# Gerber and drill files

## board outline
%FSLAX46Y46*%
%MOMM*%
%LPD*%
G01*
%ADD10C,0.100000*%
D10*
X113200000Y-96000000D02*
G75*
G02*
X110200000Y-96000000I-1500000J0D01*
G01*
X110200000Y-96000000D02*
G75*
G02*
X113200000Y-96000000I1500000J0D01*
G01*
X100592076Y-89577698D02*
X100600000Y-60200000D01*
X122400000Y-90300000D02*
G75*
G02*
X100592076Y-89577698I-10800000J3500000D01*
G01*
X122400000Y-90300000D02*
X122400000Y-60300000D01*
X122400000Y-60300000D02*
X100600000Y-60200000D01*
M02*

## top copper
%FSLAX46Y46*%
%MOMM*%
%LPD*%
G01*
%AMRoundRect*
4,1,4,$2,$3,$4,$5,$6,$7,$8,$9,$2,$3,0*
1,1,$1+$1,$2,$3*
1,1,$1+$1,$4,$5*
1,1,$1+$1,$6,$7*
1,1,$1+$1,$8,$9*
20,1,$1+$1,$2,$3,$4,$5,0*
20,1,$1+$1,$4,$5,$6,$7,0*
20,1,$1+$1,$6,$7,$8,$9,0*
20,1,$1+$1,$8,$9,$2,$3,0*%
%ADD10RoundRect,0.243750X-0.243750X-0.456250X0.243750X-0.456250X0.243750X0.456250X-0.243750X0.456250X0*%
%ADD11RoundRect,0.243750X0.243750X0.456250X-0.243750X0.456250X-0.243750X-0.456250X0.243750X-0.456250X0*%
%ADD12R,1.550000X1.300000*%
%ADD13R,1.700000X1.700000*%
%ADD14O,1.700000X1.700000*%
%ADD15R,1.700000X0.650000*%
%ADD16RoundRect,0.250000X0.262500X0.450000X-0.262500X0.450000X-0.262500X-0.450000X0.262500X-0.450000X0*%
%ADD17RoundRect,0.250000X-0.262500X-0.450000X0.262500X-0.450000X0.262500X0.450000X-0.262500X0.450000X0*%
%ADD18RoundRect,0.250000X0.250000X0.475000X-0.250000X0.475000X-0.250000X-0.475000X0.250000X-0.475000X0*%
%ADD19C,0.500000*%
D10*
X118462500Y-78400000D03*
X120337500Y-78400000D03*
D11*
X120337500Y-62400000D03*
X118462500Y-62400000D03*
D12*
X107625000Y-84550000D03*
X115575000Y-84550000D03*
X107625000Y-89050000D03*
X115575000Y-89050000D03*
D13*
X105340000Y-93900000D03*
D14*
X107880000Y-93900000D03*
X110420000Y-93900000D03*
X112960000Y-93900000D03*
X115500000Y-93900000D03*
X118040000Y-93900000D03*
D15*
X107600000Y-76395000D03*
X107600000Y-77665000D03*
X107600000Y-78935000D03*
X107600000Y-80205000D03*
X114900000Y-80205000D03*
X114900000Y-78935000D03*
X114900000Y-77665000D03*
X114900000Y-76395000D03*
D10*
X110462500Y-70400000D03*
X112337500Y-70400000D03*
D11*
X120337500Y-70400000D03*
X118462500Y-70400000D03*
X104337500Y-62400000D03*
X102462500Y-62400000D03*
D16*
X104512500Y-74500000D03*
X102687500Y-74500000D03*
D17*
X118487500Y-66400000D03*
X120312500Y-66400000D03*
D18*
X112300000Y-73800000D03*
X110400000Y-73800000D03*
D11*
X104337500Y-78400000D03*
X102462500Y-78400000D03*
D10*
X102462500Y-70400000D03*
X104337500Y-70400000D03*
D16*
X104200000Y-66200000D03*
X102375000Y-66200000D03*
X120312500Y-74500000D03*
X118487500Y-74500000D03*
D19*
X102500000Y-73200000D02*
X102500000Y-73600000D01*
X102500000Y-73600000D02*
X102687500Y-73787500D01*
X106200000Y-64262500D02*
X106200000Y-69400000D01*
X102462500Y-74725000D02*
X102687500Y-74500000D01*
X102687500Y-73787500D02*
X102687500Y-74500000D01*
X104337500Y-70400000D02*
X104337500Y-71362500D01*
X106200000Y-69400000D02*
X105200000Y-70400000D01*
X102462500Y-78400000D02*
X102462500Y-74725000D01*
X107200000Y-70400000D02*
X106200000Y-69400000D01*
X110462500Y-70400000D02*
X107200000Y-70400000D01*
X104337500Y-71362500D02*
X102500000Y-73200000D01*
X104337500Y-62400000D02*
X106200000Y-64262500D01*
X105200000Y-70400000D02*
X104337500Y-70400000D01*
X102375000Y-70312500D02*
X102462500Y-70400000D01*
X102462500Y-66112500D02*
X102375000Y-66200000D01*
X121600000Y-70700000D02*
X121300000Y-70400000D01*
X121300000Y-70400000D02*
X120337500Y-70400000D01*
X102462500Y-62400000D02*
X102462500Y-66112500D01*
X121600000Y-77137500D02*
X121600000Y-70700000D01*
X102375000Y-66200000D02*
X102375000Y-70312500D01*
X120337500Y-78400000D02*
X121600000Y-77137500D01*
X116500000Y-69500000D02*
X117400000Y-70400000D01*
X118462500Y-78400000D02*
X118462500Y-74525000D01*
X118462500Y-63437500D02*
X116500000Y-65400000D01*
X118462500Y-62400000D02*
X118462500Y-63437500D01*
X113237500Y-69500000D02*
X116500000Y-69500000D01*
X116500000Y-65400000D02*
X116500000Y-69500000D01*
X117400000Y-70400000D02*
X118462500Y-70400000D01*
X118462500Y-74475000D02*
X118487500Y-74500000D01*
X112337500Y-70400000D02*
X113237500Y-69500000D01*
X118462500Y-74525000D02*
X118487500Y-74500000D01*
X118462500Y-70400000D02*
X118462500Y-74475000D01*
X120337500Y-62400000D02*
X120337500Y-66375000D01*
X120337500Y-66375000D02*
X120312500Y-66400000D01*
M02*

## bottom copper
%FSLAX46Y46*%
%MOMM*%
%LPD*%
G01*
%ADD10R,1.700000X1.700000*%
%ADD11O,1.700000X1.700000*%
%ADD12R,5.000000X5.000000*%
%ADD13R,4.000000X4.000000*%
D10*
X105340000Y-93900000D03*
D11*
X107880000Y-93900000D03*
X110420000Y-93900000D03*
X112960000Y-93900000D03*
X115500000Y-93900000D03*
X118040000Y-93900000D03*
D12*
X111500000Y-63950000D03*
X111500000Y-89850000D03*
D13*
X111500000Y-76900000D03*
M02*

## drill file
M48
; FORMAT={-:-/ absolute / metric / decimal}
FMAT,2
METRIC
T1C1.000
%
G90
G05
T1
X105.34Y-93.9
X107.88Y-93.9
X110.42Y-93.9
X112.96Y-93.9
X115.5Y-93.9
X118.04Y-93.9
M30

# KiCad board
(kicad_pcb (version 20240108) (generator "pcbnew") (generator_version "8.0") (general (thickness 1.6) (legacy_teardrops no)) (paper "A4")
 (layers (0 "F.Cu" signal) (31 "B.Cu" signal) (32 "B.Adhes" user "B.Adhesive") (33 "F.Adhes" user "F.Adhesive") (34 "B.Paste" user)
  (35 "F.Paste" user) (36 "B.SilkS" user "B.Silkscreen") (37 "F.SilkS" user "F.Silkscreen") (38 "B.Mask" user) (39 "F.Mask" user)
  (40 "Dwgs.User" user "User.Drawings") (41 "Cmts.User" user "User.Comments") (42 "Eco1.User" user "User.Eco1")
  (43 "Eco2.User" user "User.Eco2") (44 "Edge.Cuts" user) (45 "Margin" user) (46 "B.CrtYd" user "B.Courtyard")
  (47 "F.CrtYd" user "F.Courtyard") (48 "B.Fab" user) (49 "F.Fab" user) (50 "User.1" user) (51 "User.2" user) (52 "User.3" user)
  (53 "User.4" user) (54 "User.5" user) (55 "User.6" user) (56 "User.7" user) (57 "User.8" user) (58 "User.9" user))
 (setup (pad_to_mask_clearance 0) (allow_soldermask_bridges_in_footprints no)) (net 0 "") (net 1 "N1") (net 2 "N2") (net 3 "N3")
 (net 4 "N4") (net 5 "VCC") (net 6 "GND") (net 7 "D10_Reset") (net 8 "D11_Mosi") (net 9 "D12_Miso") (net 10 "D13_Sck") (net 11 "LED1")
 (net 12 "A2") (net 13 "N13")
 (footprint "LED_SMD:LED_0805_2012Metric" (layer "F.Cu") (at 119.4 78.4)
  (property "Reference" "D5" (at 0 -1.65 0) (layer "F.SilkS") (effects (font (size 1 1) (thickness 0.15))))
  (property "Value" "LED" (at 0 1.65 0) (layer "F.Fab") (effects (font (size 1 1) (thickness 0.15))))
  (pad "1" smd roundrect (at -0.9375 0) (size 0.975 1.4) (layers "F.Cu" "F.Paste" "F.Mask") (roundrect_rratio 0.25) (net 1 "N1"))
  (pad "2" smd roundrect (at 0.9375 0) (size 0.975 1.4) (layers "F.Cu" "F.Paste" "F.Mask") (roundrect_rratio 0.25) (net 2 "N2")))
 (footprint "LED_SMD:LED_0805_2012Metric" (layer "F.Cu") (at 119.4 62.4 180)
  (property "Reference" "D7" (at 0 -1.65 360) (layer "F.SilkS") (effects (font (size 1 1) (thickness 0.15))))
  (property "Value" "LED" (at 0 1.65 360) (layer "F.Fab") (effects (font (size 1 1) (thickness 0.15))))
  (pad "1" smd roundrect (at -0.9375 0 180) (size 0.975 1.4) (layers "F.Cu" "F.Paste" "F.Mask") (roundrect_rratio 0.25) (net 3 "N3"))
  (pad "2" smd roundrect (at 0.9375 0 180) (size 0.975 1.4) (layers "F.Cu" "F.Paste" "F.Mask") (roundrect_rratio 0.25) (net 1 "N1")))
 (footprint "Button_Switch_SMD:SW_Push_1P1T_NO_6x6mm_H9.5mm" (layer "F.Cu") (at 111.6 86.8)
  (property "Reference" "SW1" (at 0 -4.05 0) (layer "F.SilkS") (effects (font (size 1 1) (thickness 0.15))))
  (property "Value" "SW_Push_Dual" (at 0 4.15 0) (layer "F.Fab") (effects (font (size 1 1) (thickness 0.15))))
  (pad "1" smd rect (at -3.975 -2.25) (size 1.55 1.3) (layers "F.Cu" "F.Paste" "F.Mask") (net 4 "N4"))
  (pad "1" smd rect (at 3.975 -2.25) (size 1.55 1.3) (layers "F.Cu" "F.Paste" "F.Mask") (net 4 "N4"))
  (pad "2" smd rect (at -3.975 2.25) (size 1.55 1.3) (layers "F.Cu" "F.Paste" "F.Mask") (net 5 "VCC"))
  (pad "2" smd rect (at 3.975 2.25) (size 1.55 1.3) (layers "F.Cu" "F.Paste" "F.Mask") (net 5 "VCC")))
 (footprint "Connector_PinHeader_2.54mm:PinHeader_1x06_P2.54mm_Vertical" (layer "F.Cu") (at 105.34 93.9 90)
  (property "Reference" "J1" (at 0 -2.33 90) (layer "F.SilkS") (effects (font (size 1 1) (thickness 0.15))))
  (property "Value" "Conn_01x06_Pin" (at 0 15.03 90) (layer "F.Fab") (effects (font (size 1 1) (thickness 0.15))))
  (pad "1" thru_hole rect (at 0 0 90) (size 1.7 1.7) (drill 1) (layers "*.Cu" "*.Mask") (remove_unused_layers no) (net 5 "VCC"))
  (pad "2" thru_hole oval (at 0 2.54 90) (size 1.7 1.7) (drill 1) (layers "*.Cu" "*.Mask") (remove_unused_layers no) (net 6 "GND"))
  (pad "3" thru_hole oval (at 0 5.08 90) (size 1.7 1.7) (drill 1) (layers "*.Cu" "*.Mask") (remove_unused_layers no) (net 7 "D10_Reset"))
  (pad "4" thru_hole oval (at 0 7.62 90) (size 1.7 1.7) (drill 1) (layers "*.Cu" "*.Mask") (remove_unused_layers no) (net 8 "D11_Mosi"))
  (pad "5" thru_hole oval (at 0 10.16 90) (size 1.7 1.7) (drill 1) (layers "*.Cu" "*.Mask") (remove_unused_layers no) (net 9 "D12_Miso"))
  (pad "6" thru_hole oval (at 0 12.7 90) (size 1.7 1.7) (drill 1) (layers "*.Cu" "*.Mask") (remove_unused_layers no) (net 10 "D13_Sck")))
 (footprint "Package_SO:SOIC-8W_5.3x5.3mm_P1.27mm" (layer "F.Cu") (at 111.25 78.3)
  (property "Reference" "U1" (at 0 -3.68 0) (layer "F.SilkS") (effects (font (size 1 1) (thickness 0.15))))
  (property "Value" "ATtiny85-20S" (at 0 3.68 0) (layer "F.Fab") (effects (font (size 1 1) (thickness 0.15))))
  (pad "1" smd rect (at -3.65 -1.905) (size 1.7 0.65) (layers "F.Cu" "F.Paste" "F.Mask") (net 7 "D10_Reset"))
  (pad "2" smd rect (at -3.65 -0.635) (size 1.7 0.65) (layers "F.Cu" "F.Paste" "F.Mask") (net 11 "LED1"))
  (pad "3" smd rect (at -3.65 0.635) (size 1.7 0.65) (layers "F.Cu" "F.Paste" "F.Mask") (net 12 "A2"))
  (pad "4" smd rect (at -3.65 1.905) (size 1.7 0.65) (layers "F.Cu" "F.Paste" "F.Mask") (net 6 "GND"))
  (pad "5" smd rect (at 3.65 1.905) (size 1.7 0.65) (layers "F.Cu" "F.Paste" "F.Mask") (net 8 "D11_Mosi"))
  (pad "6" smd rect (at 3.65 0.635) (size 1.7 0.65) (layers "F.Cu" "F.Paste" "F.Mask") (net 9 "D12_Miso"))
  (pad "7" smd rect (at 3.65 -0.635) (size 1.7 0.65) (layers "F.Cu" "F.Paste" "F.Mask") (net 10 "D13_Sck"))
  (pad "8" smd rect (at 3.65 -1.905) (size 1.7 0.65) (layers "F.Cu" "F.Paste" "F.Mask") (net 5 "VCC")))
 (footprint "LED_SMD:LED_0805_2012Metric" (layer "F.Cu") (at 111.4 70.4)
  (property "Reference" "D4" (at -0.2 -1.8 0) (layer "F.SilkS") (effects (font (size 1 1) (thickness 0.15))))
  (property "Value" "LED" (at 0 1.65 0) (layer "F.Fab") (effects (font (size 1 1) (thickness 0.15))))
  (pad "1" smd roundrect (at -0.9375 0) (size 0.975 1.4) (layers "F.Cu" "F.Paste" "F.Mask") (roundrect_rratio 0.25) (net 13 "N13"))
  (pad "2" smd roundrect (at 0.9375 0) (size 0.975 1.4) (layers "F.Cu" "F.Paste" "F.Mask") (roundrect_rratio 0.25) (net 1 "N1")))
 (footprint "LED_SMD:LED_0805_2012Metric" (layer "F.Cu") (at 119.4 70.4 180)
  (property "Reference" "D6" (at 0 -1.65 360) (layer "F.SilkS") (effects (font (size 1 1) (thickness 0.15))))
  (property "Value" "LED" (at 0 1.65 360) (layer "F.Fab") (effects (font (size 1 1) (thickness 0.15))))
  (pad "1" smd roundrect (at -0.9375 0 180) (size 0.975 1.4) (layers "F.Cu" "F.Paste" "F.Mask") (roundrect_rratio 0.25) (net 2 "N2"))
  (pad "2" smd roundrect (at 0.9375 0 180) (size 0.975 1.4) (layers "F.Cu" "F.Paste" "F.Mask") (roundrect_rratio 0.25) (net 1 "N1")))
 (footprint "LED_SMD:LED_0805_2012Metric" (layer "F.Cu") (at 103.4 62.4 180)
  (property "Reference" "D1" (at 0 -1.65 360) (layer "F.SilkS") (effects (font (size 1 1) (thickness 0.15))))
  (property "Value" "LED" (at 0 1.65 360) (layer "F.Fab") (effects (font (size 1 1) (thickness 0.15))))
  (pad "1" smd roundrect (at -0.9375 0 180) (size 0.975 1.4) (layers "F.Cu" "F.Paste" "F.Mask") (roundrect_rratio 0.25) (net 13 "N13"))
  (pad "2" smd roundrect (at 0.9375 0 180) (size 0.975 1.4) (layers "F.Cu" "F.Paste" "F.Mask") (roundrect_rratio 0.25) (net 2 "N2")))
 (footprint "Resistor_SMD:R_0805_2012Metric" (layer "F.Cu") (at 103.6 74.5 180)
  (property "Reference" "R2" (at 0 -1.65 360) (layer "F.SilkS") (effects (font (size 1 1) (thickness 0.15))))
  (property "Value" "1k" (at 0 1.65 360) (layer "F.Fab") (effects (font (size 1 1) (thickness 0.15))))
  (pad "1" smd roundrect (at -0.9125 0 180) (size 1.025 1.4) (layers "F.Cu" "F.Paste" "F.Mask") (roundrect_rratio 0.243902)
   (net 8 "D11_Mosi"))
  (pad "2" smd roundrect (at 0.9125 0 180) (size 1.025 1.4) (layers "F.Cu" "F.Paste" "F.Mask") (roundrect_rratio 0.243902) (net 13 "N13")))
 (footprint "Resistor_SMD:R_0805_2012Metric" (layer "F.Cu") (at 119.4 66.4)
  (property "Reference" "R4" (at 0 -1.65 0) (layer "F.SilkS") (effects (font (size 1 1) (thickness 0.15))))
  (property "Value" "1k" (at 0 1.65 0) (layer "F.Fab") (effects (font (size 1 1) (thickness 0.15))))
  (pad "1" smd roundrect (at -0.9125 0) (size 1.025 1.4) (layers "F.Cu" "F.Paste" "F.Mask") (roundrect_rratio 0.243902) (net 10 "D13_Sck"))
  (pad "2" smd roundrect (at 0.9125 0) (size 1.025 1.4) (layers "F.Cu" "F.Paste" "F.Mask") (roundrect_rratio 0.243902) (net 3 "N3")))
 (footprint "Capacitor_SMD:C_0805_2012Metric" (layer "F.Cu") (at 111.35 73.8 180)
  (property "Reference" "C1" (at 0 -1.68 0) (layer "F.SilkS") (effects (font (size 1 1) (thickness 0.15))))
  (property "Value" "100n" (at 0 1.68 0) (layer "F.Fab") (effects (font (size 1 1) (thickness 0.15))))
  (pad "1" smd roundrect (at -0.95 0 180) (size 1 1.45) (layers "F.Cu" "F.Paste" "F.Mask") (roundrect_rratio 0.25) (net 5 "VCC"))
  (pad "2" smd roundrect (at 0.95 0 180) (size 1 1.45) (layers "F.Cu" "F.Paste" "F.Mask") (roundrect_rratio 0.25) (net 6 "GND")))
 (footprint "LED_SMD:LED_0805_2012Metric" (layer "F.Cu") (at 103.4 78.4 180)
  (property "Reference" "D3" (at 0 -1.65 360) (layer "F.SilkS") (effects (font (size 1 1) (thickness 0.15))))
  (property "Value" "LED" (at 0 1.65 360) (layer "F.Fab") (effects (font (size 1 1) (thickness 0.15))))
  (pad "1" smd roundrect (at -0.9375 0 180) (size 0.975 1.4) (layers "F.Cu" "F.Paste" "F.Mask") (roundrect_rratio 0.25) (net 1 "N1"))
  (pad "2" smd roundrect (at 0.9375 0 180) (size 0.975 1.4) (layers "F.Cu" "F.Paste" "F.Mask") (roundrect_rratio 0.25) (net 13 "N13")))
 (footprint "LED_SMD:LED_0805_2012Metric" (layer "F.Cu") (at 103.4 70.4)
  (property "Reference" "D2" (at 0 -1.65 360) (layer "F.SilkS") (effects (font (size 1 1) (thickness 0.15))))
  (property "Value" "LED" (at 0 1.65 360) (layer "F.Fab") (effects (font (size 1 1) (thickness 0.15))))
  (pad "1" smd roundrect (at -0.9375 0) (size 0.975 1.4) (layers "F.Cu" "F.Paste" "F.Mask") (roundrect_rratio 0.25) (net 2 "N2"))
  (pad "2" smd roundrect (at 0.9375 0) (size 0.975 1.4) (layers "F.Cu" "F.Paste" "F.Mask") (roundrect_rratio 0.25) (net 13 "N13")))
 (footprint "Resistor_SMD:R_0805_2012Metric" (layer "F.Cu") (at 103.2875 66.2 180)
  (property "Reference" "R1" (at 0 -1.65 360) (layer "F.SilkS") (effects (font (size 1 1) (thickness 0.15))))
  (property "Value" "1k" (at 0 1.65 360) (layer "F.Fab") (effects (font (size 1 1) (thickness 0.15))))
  (pad "1" smd roundrect (at -0.9125 0 180) (size 1.025 1.4) (layers "F.Cu" "F.Paste" "F.Mask") (roundrect_rratio 0.243902) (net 11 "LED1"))
  (pad "2" smd roundrect (at 0.9125 0 180) (size 1.025 1.4) (layers "F.Cu" "F.Paste" "F.Mask") (roundrect_rratio 0.243902) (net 2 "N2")))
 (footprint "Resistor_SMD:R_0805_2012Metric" (layer "F.Cu") (at 119.4 74.5 180)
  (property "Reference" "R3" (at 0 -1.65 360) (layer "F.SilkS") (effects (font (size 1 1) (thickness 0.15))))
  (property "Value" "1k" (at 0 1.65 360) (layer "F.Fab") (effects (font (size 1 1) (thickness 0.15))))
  (pad "1" smd roundrect (at -0.9125 0 180) (size 1.025 1.4) (layers "F.Cu" "F.Paste" "F.Mask") (roundrect_rratio 0.243902)
   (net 9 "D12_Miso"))
  (pad "2" smd roundrect (at 0.9125 0 180) (size 1.025 1.4) (layers "F.Cu" "F.Paste" "F.Mask") (roundrect_rratio 0.243902) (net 1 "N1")))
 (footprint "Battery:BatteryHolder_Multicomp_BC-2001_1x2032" (layer "B.Cu") (at 111.5 76.9 -90)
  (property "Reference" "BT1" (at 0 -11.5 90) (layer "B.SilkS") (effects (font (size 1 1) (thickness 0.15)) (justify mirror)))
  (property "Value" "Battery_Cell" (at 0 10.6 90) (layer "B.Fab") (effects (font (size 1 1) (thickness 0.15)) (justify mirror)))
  (pad "1" smd rect (at -12.95 0 270) (size 5 5) (layers "B.Cu" "B.Paste" "B.Mask") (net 4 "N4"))
  (pad "1" smd rect (at 12.95 0 270) (size 5 5) (layers "B.Cu" "B.Paste" "B.Mask") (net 4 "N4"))
  (pad "2" smd rect (at 0 0 270) (size 4 4) (layers "B.Cu" "B.Paste" "B.Mask") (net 6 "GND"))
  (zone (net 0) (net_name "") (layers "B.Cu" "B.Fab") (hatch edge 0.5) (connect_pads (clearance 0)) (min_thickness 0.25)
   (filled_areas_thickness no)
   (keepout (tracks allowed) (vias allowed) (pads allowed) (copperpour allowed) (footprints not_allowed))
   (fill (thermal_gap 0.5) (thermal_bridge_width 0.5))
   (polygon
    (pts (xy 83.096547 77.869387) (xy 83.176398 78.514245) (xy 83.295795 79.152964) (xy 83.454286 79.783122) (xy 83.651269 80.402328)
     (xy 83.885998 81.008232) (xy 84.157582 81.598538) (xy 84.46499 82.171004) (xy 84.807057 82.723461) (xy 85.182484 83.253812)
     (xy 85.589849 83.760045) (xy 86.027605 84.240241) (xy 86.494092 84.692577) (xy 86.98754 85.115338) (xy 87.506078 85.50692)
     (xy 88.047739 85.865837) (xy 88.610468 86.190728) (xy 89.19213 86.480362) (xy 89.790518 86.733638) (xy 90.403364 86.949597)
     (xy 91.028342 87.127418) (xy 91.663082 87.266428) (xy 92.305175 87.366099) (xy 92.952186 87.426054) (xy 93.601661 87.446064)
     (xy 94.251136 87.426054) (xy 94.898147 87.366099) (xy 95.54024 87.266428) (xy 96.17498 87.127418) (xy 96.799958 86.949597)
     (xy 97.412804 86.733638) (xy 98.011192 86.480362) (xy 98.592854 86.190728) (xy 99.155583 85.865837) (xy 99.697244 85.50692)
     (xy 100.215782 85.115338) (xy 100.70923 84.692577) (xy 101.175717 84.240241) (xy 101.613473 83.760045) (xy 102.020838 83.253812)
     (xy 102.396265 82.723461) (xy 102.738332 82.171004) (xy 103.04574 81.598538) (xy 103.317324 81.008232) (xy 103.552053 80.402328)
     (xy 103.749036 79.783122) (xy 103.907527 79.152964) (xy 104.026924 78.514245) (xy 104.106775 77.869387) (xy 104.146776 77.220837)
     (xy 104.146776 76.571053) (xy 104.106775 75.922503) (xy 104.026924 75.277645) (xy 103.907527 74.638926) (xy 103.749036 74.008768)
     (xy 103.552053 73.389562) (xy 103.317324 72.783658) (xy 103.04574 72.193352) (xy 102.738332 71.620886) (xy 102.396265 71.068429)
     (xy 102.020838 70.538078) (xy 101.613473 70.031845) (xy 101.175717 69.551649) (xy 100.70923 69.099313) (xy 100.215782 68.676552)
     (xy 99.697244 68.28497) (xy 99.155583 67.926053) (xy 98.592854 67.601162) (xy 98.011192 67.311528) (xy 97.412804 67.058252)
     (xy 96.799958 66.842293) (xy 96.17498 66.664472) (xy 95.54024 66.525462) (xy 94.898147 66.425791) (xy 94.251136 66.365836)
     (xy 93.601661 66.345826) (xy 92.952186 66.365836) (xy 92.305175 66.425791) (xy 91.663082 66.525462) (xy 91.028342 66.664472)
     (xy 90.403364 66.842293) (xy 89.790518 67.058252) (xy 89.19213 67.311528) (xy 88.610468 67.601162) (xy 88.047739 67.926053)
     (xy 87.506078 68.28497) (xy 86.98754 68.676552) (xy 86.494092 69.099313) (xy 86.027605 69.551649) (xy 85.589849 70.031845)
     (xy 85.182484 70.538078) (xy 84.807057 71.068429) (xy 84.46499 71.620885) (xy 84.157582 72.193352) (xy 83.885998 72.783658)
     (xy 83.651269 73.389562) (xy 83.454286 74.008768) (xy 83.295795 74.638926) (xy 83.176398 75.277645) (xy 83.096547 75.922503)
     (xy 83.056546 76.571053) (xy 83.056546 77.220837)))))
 (gr_circle (center 111.7 96) (end 113.2 96) (stroke (width 0.1) (type default)) (fill none) (layer "Edge.Cuts"))
 (gr_line (start 100.592076 89.577698) (end 100.6 60.2) (stroke (width 0.1) (type default)) (layer "Edge.Cuts"))
 (gr_arc (start 122.4 90.3) (mid 111.224183 98.14675) (end 100.592076 89.577698) (stroke (width 0.1) (type default)) (layer "Edge.Cuts"))
 (gr_line (start 122.4 90.3) (end 122.4 60.3) (stroke (width 0.1) (type default)) (layer "Edge.Cuts"))
 (gr_line (start 122.4 60.3) (end 100.6 60.2) (stroke (width 0.1) (type default)) (layer "Edge.Cuts"))
 (segment (start 102.5 73.2) (end 102.5 73.6) (width 0.5) (layer "F.Cu") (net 13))
 (segment (start 102.5 73.6) (end 102.6875 73.7875) (width 0.5) (layer "F.Cu") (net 13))
 (segment (start 106.2 64.2625) (end 106.2 69.4) (width 0.5) (layer "F.Cu") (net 13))
 (segment (start 102.4625 74.725) (end 102.6875 74.5) (width 0.5) (layer "F.Cu") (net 13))
 (segment (start 102.6875 73.7875) (end 102.6875 74.5) (width 0.5) (layer "F.Cu") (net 13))
 (segment (start 104.3375 70.4) (end 104.3375 71.3625) (width 0.5) (layer "F.Cu") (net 13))
 (segment (start 106.2 69.4) (end 105.2 70.4) (width 0.5) (layer "F.Cu") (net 13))
 (segment (start 102.4625 78.4) (end 102.4625 74.725) (width 0.5) (layer "F.Cu") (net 13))
 (segment (start 107.2 70.4) (end 106.2 69.4) (width 0.5) (layer "F.Cu") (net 13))
 (segment (start 110.4625 70.4) (end 107.2 70.4) (width 0.5) (layer "F.Cu") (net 13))
 (segment (start 104.3375 71.3625) (end 102.5 73.2) (width 0.5) (layer "F.Cu") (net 13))
 (segment (start 104.3375 62.4) (end 106.2 64.2625) (width 0.5) (layer "F.Cu") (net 13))
 (segment (start 105.2 70.4) (end 104.3375 70.4) (width 0.5) (layer "F.Cu") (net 13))
 (segment (start 102.375 70.3125) (end 102.4625 70.4) (width 0.5) (layer "F.Cu") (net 2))
 (segment (start 102.4625 66.1125) (end 102.375 66.2) (width 0.5) (layer "F.Cu") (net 2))
 (segment (start 121.6 70.7) (end 121.3 70.4) (width 0.5) (layer "F.Cu") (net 2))
 (segment (start 121.3 70.4) (end 120.3375 70.4) (width 0.5) (layer "F.Cu") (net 2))
 (segment (start 102.4625 62.4) (end 102.4625 66.1125) (width 0.5) (layer "F.Cu") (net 2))
 (segment (start 121.6 77.1375) (end 121.6 70.7) (width 0.5) (layer "F.Cu") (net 2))
 (segment (start 102.375 66.2) (end 102.375 70.3125) (width 0.5) (layer "F.Cu") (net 2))
 (segment (start 120.3375 78.4) (end 121.6 77.1375) (width 0.5) (layer "F.Cu") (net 2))
 (segment (start 116.5 69.5) (end 117.4 70.4) (width 0.5) (layer "F.Cu") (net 1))
 (segment (start 118.4625 78.4) (end 118.4625 74.525) (width 0.5) (layer "F.Cu") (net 1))
 (segment (start 118.4625 63.4375) (end 116.5 65.4) (width 0.5) (layer "F.Cu") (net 1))
 (segment (start 118.4625 62.4) (end 118.4625 63.4375) (width 0.5) (layer "F.Cu") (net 1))
 (segment (start 113.2375 69.5) (end 116.5 69.5) (width 0.5) (layer "F.Cu") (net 1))
 (segment (start 116.5 65.4) (end 116.5 69.5) (width 0.5) (layer "F.Cu") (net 1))
 (segment (start 117.4 70.4) (end 118.4625 70.4) (width 0.5) (layer "F.Cu") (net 1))
 (segment (start 118.4625 74.475) (end 118.4875 74.5) (width 0.5) (layer "F.Cu") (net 1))
 (segment (start 112.3375 70.4) (end 113.2375 69.5) (width 0.5) (layer "F.Cu") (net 1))
 (segment (start 118.4625 74.525) (end 118.4875 74.5) (width 0.5) (layer "F.Cu") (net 1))
 (segment (start 118.4625 70.4) (end 118.4625 74.475) (width 0.5) (layer "F.Cu") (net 1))
 (segment (start 120.3375 62.4) (end 120.3375 66.375) (width 0.5) (layer "F.Cu") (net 3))
 (segment (start 120.3375 66.375) (end 120.3125 66.4) (width 0.5) (layer "F.Cu") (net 3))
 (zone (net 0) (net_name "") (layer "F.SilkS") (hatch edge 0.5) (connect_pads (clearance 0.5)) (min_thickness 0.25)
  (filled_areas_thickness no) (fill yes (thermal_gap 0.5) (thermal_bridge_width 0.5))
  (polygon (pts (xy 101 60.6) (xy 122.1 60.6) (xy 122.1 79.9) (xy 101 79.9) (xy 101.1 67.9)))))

